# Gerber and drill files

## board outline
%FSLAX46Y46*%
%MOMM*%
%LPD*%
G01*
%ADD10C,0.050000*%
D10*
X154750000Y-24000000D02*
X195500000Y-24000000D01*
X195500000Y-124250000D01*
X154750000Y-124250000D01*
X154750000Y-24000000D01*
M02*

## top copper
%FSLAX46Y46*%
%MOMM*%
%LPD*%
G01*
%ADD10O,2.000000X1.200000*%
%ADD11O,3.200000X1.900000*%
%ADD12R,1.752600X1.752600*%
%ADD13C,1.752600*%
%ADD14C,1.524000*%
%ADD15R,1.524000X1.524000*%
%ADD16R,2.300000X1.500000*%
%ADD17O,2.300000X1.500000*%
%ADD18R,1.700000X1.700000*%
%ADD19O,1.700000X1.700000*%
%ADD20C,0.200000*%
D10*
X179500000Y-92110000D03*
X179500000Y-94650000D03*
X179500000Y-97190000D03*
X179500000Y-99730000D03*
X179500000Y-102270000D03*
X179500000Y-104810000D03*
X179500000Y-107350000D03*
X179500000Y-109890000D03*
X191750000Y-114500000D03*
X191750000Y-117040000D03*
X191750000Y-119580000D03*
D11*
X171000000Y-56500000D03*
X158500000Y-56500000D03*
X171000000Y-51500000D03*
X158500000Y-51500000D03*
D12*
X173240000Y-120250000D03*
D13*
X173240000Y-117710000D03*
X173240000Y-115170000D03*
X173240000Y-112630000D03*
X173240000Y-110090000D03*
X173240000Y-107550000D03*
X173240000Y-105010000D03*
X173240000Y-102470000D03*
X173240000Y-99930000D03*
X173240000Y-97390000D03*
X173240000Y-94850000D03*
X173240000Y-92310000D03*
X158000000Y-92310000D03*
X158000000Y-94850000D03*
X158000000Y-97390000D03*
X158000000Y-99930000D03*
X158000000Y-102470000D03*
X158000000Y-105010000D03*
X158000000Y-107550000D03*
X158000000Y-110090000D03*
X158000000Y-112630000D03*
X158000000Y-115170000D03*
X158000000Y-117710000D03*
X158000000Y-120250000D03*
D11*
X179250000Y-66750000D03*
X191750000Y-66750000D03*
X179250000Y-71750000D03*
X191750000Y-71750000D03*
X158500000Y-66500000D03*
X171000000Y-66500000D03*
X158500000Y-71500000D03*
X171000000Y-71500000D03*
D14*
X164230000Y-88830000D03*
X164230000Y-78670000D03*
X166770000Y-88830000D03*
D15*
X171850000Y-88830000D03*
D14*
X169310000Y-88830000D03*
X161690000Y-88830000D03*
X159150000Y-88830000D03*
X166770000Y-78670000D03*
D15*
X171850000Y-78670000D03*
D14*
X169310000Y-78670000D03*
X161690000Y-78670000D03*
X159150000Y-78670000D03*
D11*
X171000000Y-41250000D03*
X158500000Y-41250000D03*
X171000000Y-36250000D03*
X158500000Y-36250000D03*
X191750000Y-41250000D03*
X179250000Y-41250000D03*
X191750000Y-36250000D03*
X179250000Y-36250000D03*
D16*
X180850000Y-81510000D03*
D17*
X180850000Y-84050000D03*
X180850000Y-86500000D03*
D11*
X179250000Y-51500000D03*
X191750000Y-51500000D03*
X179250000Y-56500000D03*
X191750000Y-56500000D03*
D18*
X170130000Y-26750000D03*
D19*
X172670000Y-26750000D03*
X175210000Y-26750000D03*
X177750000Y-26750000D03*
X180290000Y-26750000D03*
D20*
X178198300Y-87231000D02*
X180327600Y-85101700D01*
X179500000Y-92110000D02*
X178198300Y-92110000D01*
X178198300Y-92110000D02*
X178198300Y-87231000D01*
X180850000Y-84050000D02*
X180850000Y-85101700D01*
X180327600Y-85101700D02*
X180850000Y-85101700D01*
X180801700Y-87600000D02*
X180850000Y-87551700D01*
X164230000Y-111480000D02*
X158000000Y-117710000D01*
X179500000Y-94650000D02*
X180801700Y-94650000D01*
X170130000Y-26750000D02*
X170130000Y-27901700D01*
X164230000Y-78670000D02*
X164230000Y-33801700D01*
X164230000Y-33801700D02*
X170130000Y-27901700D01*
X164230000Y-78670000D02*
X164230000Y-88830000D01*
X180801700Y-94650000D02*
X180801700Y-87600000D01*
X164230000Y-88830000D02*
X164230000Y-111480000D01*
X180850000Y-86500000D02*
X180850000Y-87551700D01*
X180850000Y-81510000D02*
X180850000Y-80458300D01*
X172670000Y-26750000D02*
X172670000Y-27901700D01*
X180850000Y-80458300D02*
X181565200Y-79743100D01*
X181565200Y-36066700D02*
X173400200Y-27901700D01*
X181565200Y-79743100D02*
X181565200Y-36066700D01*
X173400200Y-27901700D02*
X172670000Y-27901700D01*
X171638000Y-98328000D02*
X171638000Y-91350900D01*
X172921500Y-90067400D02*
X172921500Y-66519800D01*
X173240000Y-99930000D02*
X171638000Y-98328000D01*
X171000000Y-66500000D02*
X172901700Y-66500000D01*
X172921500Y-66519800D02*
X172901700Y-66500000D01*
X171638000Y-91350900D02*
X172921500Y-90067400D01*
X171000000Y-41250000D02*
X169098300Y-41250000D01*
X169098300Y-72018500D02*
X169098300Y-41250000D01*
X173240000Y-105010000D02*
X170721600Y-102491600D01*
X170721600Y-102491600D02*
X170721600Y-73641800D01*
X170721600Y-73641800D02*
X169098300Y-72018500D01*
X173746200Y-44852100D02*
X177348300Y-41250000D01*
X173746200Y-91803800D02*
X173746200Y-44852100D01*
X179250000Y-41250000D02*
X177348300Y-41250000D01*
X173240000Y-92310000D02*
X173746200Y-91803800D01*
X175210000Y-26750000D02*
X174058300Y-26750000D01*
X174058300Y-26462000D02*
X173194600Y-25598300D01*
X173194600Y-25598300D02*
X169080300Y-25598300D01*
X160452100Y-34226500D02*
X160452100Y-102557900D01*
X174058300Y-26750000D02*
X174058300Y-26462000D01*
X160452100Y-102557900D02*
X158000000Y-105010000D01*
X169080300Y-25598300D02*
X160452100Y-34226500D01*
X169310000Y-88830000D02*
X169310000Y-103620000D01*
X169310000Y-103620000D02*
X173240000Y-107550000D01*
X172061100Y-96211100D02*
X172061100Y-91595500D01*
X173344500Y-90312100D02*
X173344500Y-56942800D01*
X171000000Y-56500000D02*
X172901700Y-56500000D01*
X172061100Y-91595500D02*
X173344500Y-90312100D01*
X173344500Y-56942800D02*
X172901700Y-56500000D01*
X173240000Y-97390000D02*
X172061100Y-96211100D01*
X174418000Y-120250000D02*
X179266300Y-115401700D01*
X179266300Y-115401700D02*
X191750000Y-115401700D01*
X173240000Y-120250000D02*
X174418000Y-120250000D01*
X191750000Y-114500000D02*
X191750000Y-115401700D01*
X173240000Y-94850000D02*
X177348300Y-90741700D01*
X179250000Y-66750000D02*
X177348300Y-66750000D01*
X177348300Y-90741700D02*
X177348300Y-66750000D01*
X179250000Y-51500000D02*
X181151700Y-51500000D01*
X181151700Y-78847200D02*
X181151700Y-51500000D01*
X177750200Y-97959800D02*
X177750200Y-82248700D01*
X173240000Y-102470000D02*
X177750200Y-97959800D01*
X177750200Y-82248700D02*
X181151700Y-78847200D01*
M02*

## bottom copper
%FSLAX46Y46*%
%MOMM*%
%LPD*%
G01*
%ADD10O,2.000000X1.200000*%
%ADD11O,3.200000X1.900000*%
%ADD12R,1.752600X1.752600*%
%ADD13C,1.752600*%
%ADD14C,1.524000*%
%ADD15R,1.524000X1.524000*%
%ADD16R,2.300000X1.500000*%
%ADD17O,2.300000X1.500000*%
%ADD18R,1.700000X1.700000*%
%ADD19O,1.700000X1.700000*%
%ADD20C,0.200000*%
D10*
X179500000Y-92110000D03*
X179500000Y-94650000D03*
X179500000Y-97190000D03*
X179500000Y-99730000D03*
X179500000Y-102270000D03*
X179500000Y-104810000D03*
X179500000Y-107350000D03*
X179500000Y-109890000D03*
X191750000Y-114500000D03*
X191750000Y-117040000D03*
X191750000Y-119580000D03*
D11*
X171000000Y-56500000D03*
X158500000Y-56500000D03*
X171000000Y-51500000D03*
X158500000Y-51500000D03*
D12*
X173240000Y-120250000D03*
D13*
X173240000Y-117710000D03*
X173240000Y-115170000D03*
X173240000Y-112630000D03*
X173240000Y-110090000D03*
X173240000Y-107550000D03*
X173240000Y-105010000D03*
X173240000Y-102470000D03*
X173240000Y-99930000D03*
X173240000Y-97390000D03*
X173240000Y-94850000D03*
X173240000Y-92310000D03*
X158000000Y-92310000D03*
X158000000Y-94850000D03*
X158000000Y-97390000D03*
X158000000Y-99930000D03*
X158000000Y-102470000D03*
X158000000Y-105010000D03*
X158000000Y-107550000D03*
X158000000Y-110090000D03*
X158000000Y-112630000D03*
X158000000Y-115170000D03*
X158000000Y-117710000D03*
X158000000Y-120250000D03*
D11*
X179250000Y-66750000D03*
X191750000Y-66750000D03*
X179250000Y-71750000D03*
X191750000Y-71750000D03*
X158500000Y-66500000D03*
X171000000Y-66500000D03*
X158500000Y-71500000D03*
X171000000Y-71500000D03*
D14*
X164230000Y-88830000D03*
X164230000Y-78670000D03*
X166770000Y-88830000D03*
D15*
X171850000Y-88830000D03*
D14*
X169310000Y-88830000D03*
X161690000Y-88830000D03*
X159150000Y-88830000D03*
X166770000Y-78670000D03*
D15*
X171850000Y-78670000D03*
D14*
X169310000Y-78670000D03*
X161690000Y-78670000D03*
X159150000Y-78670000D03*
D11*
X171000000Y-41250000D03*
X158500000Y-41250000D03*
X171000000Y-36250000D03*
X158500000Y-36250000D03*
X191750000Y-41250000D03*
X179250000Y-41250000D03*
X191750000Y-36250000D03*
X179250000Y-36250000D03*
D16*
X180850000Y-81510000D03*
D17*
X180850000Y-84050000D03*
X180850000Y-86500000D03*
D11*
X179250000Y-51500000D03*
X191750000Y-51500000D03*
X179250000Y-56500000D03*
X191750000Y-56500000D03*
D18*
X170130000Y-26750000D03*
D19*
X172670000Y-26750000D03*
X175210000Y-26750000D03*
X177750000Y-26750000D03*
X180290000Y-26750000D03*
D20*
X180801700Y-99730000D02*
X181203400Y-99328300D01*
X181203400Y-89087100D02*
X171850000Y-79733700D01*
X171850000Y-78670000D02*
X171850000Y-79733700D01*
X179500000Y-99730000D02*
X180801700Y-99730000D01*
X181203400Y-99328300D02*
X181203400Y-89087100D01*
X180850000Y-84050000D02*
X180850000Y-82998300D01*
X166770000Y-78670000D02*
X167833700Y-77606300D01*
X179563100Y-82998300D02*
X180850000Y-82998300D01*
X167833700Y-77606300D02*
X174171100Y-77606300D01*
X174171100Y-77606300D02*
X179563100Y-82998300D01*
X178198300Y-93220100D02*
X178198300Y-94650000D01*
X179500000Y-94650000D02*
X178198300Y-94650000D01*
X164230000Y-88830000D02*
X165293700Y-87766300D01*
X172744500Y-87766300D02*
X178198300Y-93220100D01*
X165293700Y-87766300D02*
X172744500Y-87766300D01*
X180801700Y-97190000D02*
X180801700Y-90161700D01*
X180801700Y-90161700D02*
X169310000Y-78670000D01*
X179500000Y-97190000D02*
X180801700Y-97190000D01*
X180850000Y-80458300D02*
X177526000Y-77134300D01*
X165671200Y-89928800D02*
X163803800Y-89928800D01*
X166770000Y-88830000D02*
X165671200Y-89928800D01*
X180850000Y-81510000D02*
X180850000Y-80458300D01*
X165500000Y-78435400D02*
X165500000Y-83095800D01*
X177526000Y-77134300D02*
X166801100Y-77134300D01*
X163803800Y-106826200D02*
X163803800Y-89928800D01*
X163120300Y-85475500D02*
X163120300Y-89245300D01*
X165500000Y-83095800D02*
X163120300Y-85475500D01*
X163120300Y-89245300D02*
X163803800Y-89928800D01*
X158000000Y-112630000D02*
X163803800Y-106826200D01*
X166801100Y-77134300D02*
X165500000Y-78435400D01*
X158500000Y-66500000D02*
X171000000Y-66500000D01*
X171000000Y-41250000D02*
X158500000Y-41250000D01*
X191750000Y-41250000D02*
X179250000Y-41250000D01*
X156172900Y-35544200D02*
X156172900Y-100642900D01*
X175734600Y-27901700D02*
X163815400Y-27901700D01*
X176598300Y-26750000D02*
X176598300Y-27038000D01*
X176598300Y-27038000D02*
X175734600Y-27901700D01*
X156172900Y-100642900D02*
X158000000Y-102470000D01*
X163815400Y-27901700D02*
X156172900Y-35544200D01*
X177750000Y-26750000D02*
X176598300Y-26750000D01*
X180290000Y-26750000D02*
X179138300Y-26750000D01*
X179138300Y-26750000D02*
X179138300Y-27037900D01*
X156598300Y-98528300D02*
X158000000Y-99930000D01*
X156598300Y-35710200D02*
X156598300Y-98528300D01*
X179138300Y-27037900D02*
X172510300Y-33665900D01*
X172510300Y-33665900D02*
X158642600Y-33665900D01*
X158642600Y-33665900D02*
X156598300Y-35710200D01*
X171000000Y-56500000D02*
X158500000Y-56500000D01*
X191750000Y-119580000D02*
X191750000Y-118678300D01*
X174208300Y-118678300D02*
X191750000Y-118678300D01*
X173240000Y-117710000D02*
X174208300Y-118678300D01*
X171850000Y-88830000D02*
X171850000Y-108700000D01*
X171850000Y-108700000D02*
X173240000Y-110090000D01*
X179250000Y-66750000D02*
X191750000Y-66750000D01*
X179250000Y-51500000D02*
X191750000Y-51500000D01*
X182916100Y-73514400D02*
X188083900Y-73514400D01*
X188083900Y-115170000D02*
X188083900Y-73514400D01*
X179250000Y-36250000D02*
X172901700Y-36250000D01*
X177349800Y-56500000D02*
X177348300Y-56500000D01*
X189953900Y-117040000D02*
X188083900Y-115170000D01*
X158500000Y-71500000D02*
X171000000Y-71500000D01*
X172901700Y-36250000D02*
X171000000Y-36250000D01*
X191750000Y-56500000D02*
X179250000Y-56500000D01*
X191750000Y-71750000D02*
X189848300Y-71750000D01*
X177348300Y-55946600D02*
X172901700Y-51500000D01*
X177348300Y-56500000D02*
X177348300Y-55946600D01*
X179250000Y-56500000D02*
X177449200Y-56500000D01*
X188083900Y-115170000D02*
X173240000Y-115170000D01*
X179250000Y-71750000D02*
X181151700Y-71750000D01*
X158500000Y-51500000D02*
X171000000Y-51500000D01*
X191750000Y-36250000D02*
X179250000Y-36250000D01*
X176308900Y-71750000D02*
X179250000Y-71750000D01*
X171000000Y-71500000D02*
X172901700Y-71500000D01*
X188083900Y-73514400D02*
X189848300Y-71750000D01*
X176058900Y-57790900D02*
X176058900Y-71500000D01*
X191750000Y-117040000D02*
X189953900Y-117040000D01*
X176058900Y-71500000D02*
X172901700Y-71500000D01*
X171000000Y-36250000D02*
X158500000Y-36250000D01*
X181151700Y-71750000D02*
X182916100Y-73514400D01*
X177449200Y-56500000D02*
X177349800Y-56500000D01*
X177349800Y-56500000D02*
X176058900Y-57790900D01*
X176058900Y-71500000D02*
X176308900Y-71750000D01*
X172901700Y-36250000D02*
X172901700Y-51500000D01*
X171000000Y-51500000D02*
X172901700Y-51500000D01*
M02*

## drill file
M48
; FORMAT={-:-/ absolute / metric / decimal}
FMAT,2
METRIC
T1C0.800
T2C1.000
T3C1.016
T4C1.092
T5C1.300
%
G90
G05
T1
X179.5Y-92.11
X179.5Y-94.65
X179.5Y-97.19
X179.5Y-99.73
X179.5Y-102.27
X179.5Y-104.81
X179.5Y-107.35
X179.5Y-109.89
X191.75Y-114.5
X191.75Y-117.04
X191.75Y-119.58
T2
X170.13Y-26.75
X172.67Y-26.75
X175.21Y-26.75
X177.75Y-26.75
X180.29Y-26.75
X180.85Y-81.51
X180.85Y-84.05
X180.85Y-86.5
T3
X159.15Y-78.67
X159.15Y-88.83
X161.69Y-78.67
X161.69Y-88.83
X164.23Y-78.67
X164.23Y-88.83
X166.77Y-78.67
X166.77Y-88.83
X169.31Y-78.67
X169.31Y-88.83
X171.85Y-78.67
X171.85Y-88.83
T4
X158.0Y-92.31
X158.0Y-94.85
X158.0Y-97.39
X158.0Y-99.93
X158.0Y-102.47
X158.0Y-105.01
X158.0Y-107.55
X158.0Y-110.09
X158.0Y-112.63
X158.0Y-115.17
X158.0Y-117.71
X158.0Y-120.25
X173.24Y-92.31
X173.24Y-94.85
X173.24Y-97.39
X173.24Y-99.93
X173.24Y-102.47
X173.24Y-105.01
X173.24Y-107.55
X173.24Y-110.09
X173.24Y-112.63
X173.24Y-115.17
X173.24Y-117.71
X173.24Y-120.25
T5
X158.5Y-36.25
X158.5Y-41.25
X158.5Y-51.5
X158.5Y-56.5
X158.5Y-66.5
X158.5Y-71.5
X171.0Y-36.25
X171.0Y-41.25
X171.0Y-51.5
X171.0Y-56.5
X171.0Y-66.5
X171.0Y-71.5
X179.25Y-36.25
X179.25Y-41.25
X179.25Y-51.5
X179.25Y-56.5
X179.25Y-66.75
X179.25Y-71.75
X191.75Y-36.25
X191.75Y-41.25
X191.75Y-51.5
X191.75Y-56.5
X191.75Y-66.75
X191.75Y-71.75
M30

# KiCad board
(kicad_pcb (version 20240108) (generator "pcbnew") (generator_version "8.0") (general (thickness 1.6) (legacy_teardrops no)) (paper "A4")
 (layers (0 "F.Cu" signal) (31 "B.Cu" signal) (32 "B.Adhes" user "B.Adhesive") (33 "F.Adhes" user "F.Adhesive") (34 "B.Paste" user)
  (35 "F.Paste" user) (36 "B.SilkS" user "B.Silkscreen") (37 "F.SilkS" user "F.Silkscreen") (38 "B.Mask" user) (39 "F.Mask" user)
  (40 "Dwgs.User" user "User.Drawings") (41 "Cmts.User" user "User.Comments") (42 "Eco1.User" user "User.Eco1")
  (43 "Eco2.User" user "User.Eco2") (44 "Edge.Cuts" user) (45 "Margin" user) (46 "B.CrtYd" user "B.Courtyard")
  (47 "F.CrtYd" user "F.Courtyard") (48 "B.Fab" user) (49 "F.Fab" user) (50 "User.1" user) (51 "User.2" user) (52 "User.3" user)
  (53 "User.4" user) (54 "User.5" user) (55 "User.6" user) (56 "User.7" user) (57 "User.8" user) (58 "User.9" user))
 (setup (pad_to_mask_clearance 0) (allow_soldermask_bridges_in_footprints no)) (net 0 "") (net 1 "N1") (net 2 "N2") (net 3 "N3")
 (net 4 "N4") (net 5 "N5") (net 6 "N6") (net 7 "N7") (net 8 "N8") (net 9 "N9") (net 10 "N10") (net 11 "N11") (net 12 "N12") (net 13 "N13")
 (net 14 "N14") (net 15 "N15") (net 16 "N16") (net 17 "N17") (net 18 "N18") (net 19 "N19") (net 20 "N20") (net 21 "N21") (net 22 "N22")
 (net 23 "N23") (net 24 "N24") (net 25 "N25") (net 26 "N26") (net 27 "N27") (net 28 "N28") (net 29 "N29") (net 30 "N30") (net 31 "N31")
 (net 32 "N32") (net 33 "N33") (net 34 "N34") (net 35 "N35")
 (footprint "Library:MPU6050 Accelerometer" (layer "F.Cu") (at 186 103.25)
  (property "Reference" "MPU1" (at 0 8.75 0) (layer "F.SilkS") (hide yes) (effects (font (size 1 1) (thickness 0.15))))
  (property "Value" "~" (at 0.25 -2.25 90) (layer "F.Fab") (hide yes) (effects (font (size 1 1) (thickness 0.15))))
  (pad "1" thru_hole oval (at -6.5 -11.14 270) (size 1.2 2) (drill 0.8) (layers "*.Cu" "*.Mask") (remove_unused_layers no) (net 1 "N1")
   (thermal_bridge_angle 45))
  (pad "2" thru_hole oval (at -6.5 -8.6 270) (size 1.2 2) (drill 0.8) (layers "*.Cu" "*.Mask") (remove_unused_layers no) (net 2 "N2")
   (thermal_bridge_angle 45))
  (pad "3" thru_hole oval (at -6.5 -6.06 270) (size 1.2 2) (drill 0.8) (layers "*.Cu" "*.Mask") (remove_unused_layers no) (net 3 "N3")
   (thermal_bridge_angle 45))
  (pad "4" thru_hole oval (at -6.5 -3.52 270) (size 1.2 2) (drill 0.8) (layers "*.Cu" "*.Mask") (remove_unused_layers no) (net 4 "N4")
   (thermal_bridge_angle 45))
  (pad "5" thru_hole oval (at -6.5 -0.98 270) (size 1.2 2) (drill 0.8) (layers "*.Cu" "*.Mask") (remove_unused_layers no) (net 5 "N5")
   (thermal_bridge_angle 45))
  (pad "6" thru_hole oval (at -6.5 1.56 270) (size 1.2 2) (drill 0.8) (layers "*.Cu" "*.Mask") (remove_unused_layers no) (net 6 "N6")
   (thermal_bridge_angle 45))
  (pad "7" thru_hole oval (at -6.5 4.1 270) (size 1.2 2) (drill 0.8) (layers "*.Cu" "*.Mask") (remove_unused_layers no) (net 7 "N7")
   (thermal_bridge_angle 45))
  (pad "8" thru_hole oval (at -6.5 6.64 270) (size 1.2 2) (drill 0.8) (layers "*.Cu" "*.Mask") (remove_unused_layers no) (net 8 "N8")
   (thermal_bridge_angle 45)))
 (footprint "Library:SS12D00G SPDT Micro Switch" (layer "F.Cu") (at 191.75 117.04 -90)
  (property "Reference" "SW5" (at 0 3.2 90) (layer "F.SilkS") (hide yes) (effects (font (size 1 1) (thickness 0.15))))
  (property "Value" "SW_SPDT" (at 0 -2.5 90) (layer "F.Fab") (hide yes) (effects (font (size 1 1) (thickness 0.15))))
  (pad "1" thru_hole oval (at -2.54 0 270) (size 1.2 2) (drill 0.8) (layers "*.Cu" "*.Mask") (remove_unused_layers no) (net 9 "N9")
   (thermal_bridge_angle 45))
  (pad "2" thru_hole oval (at 0 0 270) (size 1.2 2) (drill 0.8) (layers "*.Cu" "*.Mask") (remove_unused_layers no) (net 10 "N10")
   (thermal_bridge_angle 45))
  (pad "3" thru_hole oval (at 2.54 0 270) (size 1.2 2) (drill 0.8) (layers "*.Cu" "*.Mask") (remove_unused_layers no) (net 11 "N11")
   (thermal_bridge_angle 45)))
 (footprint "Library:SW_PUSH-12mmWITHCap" (layer "F.Cu") (at 171 56.5 180)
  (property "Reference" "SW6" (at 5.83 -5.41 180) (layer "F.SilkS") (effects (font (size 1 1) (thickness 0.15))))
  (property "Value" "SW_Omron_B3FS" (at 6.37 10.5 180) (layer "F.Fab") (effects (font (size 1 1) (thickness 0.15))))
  (pad "1" thru_hole oval (at 0 0 180) (size 3.2 1.9) (drill 1.3) (layers "*.Cu" "*.Mask") (remove_unused_layers no) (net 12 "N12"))
  (pad "1" thru_hole oval (at 12.5 0 180) (size 3.2 1.9) (drill 1.3) (layers "*.Cu" "*.Mask") (remove_unused_layers no) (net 12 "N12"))
  (pad "2" thru_hole oval (at 0 5 180) (size 3.2 1.9) (drill 1.3) (layers "*.Cu" "*.Mask") (remove_unused_layers no) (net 10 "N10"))
  (pad "2" thru_hole oval (at 12.5 5 180) (size 3.2 1.9) (drill 1.3) (layers "*.Cu" "*.Mask") (remove_unused_layers no) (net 10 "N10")))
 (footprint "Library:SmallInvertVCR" (layer "F.Cu") (at 182.25 117.5)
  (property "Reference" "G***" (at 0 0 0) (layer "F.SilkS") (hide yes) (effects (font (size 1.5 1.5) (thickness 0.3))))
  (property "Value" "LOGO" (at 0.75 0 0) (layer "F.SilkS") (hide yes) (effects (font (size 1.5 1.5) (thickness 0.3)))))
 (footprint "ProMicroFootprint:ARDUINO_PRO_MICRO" (layer "F.Cu") (at 165.62 106.28 90)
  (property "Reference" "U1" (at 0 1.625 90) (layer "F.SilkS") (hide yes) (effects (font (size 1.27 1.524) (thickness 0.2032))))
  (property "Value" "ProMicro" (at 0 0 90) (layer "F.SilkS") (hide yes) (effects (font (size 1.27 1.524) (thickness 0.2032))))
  (pad "1" thru_hole rect (at -13.97 7.62 90) (size 1.7526 1.7526) (drill 1.0922) (layers "*.Cu" "*.SilkS" "*.Mask")
   (remove_unused_layers no) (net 9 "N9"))
  (pad "2" thru_hole circle (at -11.43 7.62 90) (size 1.7526 1.7526) (drill 1.0922) (layers "*.Cu" "*.SilkS" "*.Mask")
   (remove_unused_layers no) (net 11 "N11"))
  (pad "3" thru_hole circle (at -8.89 7.62 90) (size 1.7526 1.7526) (drill 1.0922) (layers "*.Cu" "*.SilkS" "*.Mask")
   (remove_unused_layers no) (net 10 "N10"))
  (pad "4" thru_hole circle (at -6.35 7.62 90) (size 1.7526 1.7526) (drill 1.0922) (layers "*.Cu" "*.SilkS" "*.Mask")
   (remove_unused_layers no) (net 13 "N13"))
  (pad "5" thru_hole circle (at -3.81 7.62 90) (size 1.7526 1.7526) (drill 1.0922) (layers "*.Cu" "*.SilkS" "*.Mask")
   (remove_unused_layers no) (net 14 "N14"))
  (pad "6" thru_hole circle (at -1.27 7.62 90) (size 1.7526 1.7526) (drill 1.0922) (layers "*.Cu" "*.SilkS" "*.Mask")
   (remove_unused_layers no) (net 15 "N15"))
  (pad "7" thru_hole circle (at 1.27 7.62 90) (size 1.7526 1.7526) (drill 1.0922) (layers "*.Cu" "*.SilkS" "*.Mask")
   (remove_unused_layers no) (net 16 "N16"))
  (pad "8" thru_hole circle (at 3.81 7.62 90) (size 1.7526 1.7526) (drill 1.0922) (layers "*.Cu" "*.SilkS" "*.Mask")
   (remove_unused_layers no) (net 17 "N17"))
  (pad "9" thru_hole circle (at 6.35 7.62 90) (size 1.7526 1.7526) (drill 1.0922) (layers "*.Cu" "*.SilkS" "*.Mask")
   (remove_unused_layers no) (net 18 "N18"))
  (pad "10" thru_hole circle (at 8.89 7.62 90) (size 1.7526 1.7526) (drill 1.0922) (layers "*.Cu" "*.SilkS" "*.Mask")
   (remove_unused_layers no) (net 12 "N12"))
  (pad "11" thru_hole circle (at 11.43 7.62 90) (size 1.7526 1.7526) (drill 1.0922) (layers "*.Cu" "*.SilkS" "*.Mask")
   (remove_unused_layers no) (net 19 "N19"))
  (pad "12" thru_hole circle (at 13.97 7.62 90) (size 1.7526 1.7526) (drill 1.0922) (layers "*.Cu" "*.SilkS" "*.Mask")
   (remove_unused_layers no) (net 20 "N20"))
  (pad "13" thru_hole circle (at 13.97 -7.62 90) (size 1.7526 1.7526) (drill 1.0922) (layers "*.Cu" "*.SilkS" "*.Mask")
   (remove_unused_layers no) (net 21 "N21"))
  (pad "14" thru_hole circle (at 11.43 -7.62 90) (size 1.7526 1.7526) (drill 1.0922) (layers "*.Cu" "*.SilkS" "*.Mask")
   (remove_unused_layers no) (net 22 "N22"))
  (pad "15" thru_hole circle (at 8.89 -7.62 90) (size 1.7526 1.7526) (drill 1.0922) (layers "*.Cu" "*.SilkS" "*.Mask")
   (remove_unused_layers no) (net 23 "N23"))
  (pad "16" thru_hole circle (at 6.35 -7.62 90) (size 1.7526 1.7526) (drill 1.0922) (layers "*.Cu" "*.SilkS" "*.Mask")
   (remove_unused_layers no) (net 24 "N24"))
  (pad "17" thru_hole circle (at 3.81 -7.62 90) (size 1.7526 1.7526) (drill 1.0922) (layers "*.Cu" "*.SilkS" "*.Mask")
   (remove_unused_layers no) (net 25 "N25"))
  (pad "18" thru_hole circle (at 1.27 -7.62 90) (size 1.7526 1.7526) (drill 1.0922) (layers "*.Cu" "*.SilkS" "*.Mask")
   (remove_unused_layers no) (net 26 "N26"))
  (pad "19" thru_hole circle (at -1.27 -7.62 90) (size 1.7526 1.7526) (drill 1.0922) (layers "*.Cu" "*.SilkS" "*.Mask")
   (remove_unused_layers no) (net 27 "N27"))
  (pad "20" thru_hole circle (at -3.81 -7.62 90) (size 1.7526 1.7526) (drill 1.0922) (layers "*.Cu" "*.SilkS" "*.Mask")
   (remove_unused_layers no) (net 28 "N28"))
  (pad "21" thru_hole circle (at -6.35 -7.62 90) (size 1.7526 1.7526) (drill 1.0922) (layers "*.Cu" "*.SilkS" "*.Mask")
   (remove_unused_layers no) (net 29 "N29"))
  (pad "22" thru_hole circle (at -8.89 -7.62 90) (size 1.7526 1.7526) (drill 1.0922) (layers "*.Cu" "*.SilkS" "*.Mask")
   (remove_unused_layers no) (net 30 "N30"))
  (pad "23" thru_hole circle (at -11.43 -7.62 90) (size 1.7526 1.7526) (drill 1.0922) (layers "*.Cu" "*.SilkS" "*.Mask")
   (remove_unused_layers no) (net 2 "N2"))
  (pad "24" thru_hole circle (at -13.97 -7.62 90) (size 1.7526 1.7526) (drill 1.0922) (layers "*.Cu" "*.SilkS" "*.Mask")
   (remove_unused_layers no) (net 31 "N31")))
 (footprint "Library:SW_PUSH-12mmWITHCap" (layer "F.Cu") (at 179.25 66.75)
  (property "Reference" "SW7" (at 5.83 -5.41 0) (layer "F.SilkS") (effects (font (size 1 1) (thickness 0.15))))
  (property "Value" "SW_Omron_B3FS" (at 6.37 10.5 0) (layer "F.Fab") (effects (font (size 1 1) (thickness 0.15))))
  (pad "1" thru_hole oval (at 0 0) (size 3.2 1.9) (drill 1.3) (layers "*.Cu" "*.Mask") (remove_unused_layers no) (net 19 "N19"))
  (pad "1" thru_hole oval (at 12.5 0) (size 3.2 1.9) (drill 1.3) (layers "*.Cu" "*.Mask") (remove_unused_layers no) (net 19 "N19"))
  (pad "2" thru_hole oval (at 0 5) (size 3.2 1.9) (drill 1.3) (layers "*.Cu" "*.Mask") (remove_unused_layers no) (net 10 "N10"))
  (pad "2" thru_hole oval (at 12.5 5) (size 3.2 1.9) (drill 1.3) (layers "*.Cu" "*.Mask") (remove_unused_layers no) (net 10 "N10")))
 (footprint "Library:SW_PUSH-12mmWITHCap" (layer "F.Cu") (at 158.5 66.5)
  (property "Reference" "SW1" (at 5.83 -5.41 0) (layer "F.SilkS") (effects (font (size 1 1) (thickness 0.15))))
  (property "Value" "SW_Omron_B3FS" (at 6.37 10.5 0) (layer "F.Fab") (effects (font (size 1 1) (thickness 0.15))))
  (pad "1" thru_hole oval (at 0 0) (size 3.2 1.9) (drill 1.3) (layers "*.Cu" "*.Mask") (remove_unused_layers no) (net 18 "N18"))
  (pad "1" thru_hole oval (at 12.5 0) (size 3.2 1.9) (drill 1.3) (layers "*.Cu" "*.Mask") (remove_unused_layers no) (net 18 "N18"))
  (pad "2" thru_hole oval (at 0 5) (size 3.2 1.9) (drill 1.3) (layers "*.Cu" "*.Mask") (remove_unused_layers no) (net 10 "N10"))
  (pad "2" thru_hole oval (at 12.5 5) (size 3.2 1.9) (drill 1.3) (layers "*.Cu" "*.Mask") (remove_unused_layers no) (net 10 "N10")))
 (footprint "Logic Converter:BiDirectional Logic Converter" (layer "F.Cu") (at 165.5 83.75 -90)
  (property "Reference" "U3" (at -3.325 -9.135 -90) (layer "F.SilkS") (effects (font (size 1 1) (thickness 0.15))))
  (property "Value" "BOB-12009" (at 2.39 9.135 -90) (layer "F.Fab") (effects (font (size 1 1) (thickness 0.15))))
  (pad "GND_1" thru_hole circle (at 5.08 1.27 270) (size 1.524 1.524) (drill 1.016) (layers "*.Cu" "*.Mask") (remove_unused_layers no)
   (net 2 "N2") (solder_mask_margin 0.102))
  (pad "GND_2" thru_hole circle (at -5.08 1.27 270) (size 1.524 1.524) (drill 1.016) (layers "*.Cu" "*.Mask") (remove_unused_layers no)
   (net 2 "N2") (solder_mask_margin 0.102))
  (pad "HV" thru_hole circle (at 5.08 -1.27 270) (size 1.524 1.524) (drill 1.016) (layers "*.Cu" "*.Mask") (remove_unused_layers no)
   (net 29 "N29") (solder_mask_margin 0.102))
  (pad "HV1" thru_hole rect (at 5.08 -6.35 270) (size 1.524 1.524) (drill 1.016) (layers "*.Cu" "*.Mask") (remove_unused_layers no)
   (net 14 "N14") (solder_mask_margin 0.102))
  (pad "HV2" thru_hole circle (at 5.08 -3.81 270) (size 1.524 1.524) (drill 1.016) (layers "*.Cu" "*.Mask") (remove_unused_layers no)
   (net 15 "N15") (solder_mask_margin 0.102))
  (pad "HV3" thru_hole circle (at 5.08 3.81 270) (size 1.524 1.524) (drill 1.016) (layers "*.Cu" "*.Mask") (remove_unused_layers no)
   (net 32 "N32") (solder_mask_margin 0.102))
  (pad "HV4" thru_hole circle (at 5.08 6.35 270) (size 1.524 1.524) (drill 1.016) (layers "*.Cu" "*.Mask") (remove_unused_layers no)
   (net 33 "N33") (solder_mask_margin 0.102))
  (pad "LV" thru_hole circle (at -5.08 -1.27 270) (size 1.524 1.524) (drill 1.016) (layers "*.Cu" "*.Mask") (remove_unused_layers no)
   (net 1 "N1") (solder_mask_margin 0.102))
  (pad "LV1" thru_hole rect (at -5.08 -6.35 270) (size 1.524 1.524) (drill 1.016) (layers "*.Cu" "*.Mask") (remove_unused_layers no)
   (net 4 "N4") (solder_mask_margin 0.102))
  (pad "LV2" thru_hole circle (at -5.08 -3.81 270) (size 1.524 1.524) (drill 1.016) (layers "*.Cu" "*.Mask") (remove_unused_layers no)
   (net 3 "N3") (solder_mask_margin 0.102))
  (pad "LV3" thru_hole circle (at -5.08 3.81 270) (size 1.524 1.524) (drill 1.016) (layers "*.Cu" "*.Mask") (remove_unused_layers no)
   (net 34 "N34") (solder_mask_margin 0.102))
  (pad "LV4" thru_hole circle (at -5.08 6.35 270) (size 1.524 1.524) (drill 1.016) (layers "*.Cu" "*.Mask") (remove_unused_layers no)
   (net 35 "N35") (solder_mask_margin 0.102)))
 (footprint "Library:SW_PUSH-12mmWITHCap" (layer "F.Cu") (at 171 41.25 180)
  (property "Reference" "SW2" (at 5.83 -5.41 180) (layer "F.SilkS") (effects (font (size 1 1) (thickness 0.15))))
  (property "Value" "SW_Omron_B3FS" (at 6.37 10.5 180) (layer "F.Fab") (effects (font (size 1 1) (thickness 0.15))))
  (pad "1" thru_hole oval (at 0 0 180) (size 3.2 1.9) (drill 1.3) (layers "*.Cu" "*.Mask") (remove_unused_layers no) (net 16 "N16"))
  (pad "1" thru_hole oval (at 12.5 0 180) (size 3.2 1.9) (drill 1.3) (layers "*.Cu" "*.Mask") (remove_unused_layers no) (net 16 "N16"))
  (pad "2" thru_hole oval (at 0 5 180) (size 3.2 1.9) (drill 1.3) (layers "*.Cu" "*.Mask") (remove_unused_layers no) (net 10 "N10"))
  (pad "2" thru_hole oval (at 12.5 5 180) (size 3.2 1.9) (drill 1.3) (layers "*.Cu" "*.Mask") (remove_unused_layers no) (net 10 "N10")))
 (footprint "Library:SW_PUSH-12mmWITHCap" (layer "F.Cu") (at 191.75 41.25 180)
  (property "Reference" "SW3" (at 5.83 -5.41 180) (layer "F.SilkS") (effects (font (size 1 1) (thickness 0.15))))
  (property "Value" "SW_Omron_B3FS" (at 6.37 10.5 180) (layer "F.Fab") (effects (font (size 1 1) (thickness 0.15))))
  (pad "1" thru_hole oval (at 0 0 180) (size 3.2 1.9) (drill 1.3) (layers "*.Cu" "*.Mask") (remove_unused_layers no) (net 20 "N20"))
  (pad "1" thru_hole oval (at 12.5 0 180) (size 3.2 1.9) (drill 1.3) (layers "*.Cu" "*.Mask") (remove_unused_layers no) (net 20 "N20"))
  (pad "2" thru_hole oval (at 0 5 180) (size 3.2 1.9) (drill 1.3) (layers "*.Cu" "*.Mask") (remove_unused_layers no) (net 10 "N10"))
  (pad "2" thru_hole oval (at 12.5 5 180) (size 3.2 1.9) (drill 1.3) (layers "*.Cu" "*.Mask") (remove_unused_layers no) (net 10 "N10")))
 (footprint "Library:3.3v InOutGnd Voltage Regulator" (layer "F.Cu") (at 179.35 84 -90)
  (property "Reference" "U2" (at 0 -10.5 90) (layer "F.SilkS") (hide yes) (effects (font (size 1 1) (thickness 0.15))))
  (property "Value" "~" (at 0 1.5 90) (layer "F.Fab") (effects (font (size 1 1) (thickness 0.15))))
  (pad "1" thru_hole rect (at -2.49 -1.5 270) (size 1.5 2.3) (drill 1) (layers "*.Cu" "*.Mask") (remove_unused_layers no) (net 29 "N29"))
  (pad "2" thru_hole oval (at 0.05 -1.5 270) (size 1.5 2.3) (drill 1) (layers "*.Cu" "*.Mask") (remove_unused_layers no) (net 1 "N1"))
  (pad "3" thru_hole oval (at 2.5 -1.5 270) (size 1.5 2.3) (drill 1) (layers "*.Cu" "*.Mask") (remove_unused_layers no) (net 2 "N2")))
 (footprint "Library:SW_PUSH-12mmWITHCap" (layer "F.Cu") (at 179.25 51.5)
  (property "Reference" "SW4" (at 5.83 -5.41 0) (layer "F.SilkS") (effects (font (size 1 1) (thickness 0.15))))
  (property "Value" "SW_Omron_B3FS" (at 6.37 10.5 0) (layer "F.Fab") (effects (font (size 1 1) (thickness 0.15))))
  (pad "1" thru_hole oval (at 0 0) (size 3.2 1.9) (drill 1.3) (layers "*.Cu" "*.Mask") (remove_unused_layers no) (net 17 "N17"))
  (pad "1" thru_hole oval (at 12.5 0) (size 3.2 1.9) (drill 1.3) (layers "*.Cu" "*.Mask") (remove_unused_layers no) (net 17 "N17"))
  (pad "2" thru_hole oval (at 0 5) (size 3.2 1.9) (drill 1.3) (layers "*.Cu" "*.Mask") (remove_unused_layers no) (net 10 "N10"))
  (pad "2" thru_hole oval (at 12.5 5) (size 3.2 1.9) (drill 1.3) (layers "*.Cu" "*.Mask") (remove_unused_layers no) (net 10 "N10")))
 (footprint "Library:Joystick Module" (layer "B.Cu") (at 170.13 26.75 -90)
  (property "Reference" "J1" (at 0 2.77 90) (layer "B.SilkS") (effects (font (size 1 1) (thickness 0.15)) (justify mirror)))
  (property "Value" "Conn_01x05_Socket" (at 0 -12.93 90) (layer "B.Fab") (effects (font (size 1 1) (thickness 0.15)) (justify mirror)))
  (pad "1" thru_hole rect (at 0 0 270) (size 1.7 1.7) (drill 1) (layers "*.Cu" "*.Mask") (remove_unused_layers no) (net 2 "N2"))
  (pad "2" thru_hole oval (at 0 -2.54 270) (size 1.7 1.7) (drill 1) (layers "*.Cu" "*.Mask") (remove_unused_layers no) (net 29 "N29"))
  (pad "3" thru_hole oval (at 0 -5.08 270) (size 1.7 1.7) (drill 1) (layers "*.Cu" "*.Mask") (remove_unused_layers no) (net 26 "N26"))
  (pad "4" thru_hole oval (at 0 -7.62 270) (size 1.7 1.7) (drill 1) (layers "*.Cu" "*.Mask") (remove_unused_layers no) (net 25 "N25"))
  (pad "5" thru_hole oval (at 0 -10.16 270) (size 1.7 1.7) (drill 1) (layers "*.Cu" "*.Mask") (remove_unused_layers no) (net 24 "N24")))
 (gr_rect (start 154.75 24) (end 195.5 124.25) (stroke (width 0.05) (type default)) (fill none) (layer "Edge.Cuts"))
 (segment (start 180.8017 99.73) (end 181.2034 99.3283) (width 0.2) (layer "B.Cu") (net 4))
 (segment (start 181.2034 89.0871) (end 171.85 79.7337) (width 0.2) (layer "B.Cu") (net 4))
 (segment (start 171.85 78.67) (end 171.85 79.7337) (width 0.2) (layer "B.Cu") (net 4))
 (segment (start 179.5 99.73) (end 180.8017 99.73) (width 0.2) (layer "B.Cu") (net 4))
 (segment (start 181.2034 99.3283) (end 181.2034 89.0871) (width 0.2) (layer "B.Cu") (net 4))
 (segment (start 178.1983 87.231) (end 180.3276 85.1017) (width 0.2) (layer "F.Cu") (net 1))
 (segment (start 179.5 92.11) (end 178.1983 92.11) (width 0.2) (layer "F.Cu") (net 1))
 (segment (start 178.1983 92.11) (end 178.1983 87.231) (width 0.2) (layer "F.Cu") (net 1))
 (segment (start 180.85 84.05) (end 180.85 85.1017) (width 0.2) (layer "F.Cu") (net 1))
 (segment (start 180.3276 85.1017) (end 180.85 85.1017) (width 0.2) (layer "F.Cu") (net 1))
 (segment (start 180.85 84.05) (end 180.85 82.9983) (width 0.2) (layer "B.Cu") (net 1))
 (segment (start 166.77 78.67) (end 167.8337 77.6063) (width 0.2) (layer "B.Cu") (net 1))
 (segment (start 179.5631 82.9983) (end 180.85 82.9983) (width 0.2) (layer "B.Cu") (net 1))
 (segment (start 167.8337 77.6063) (end 174.1711 77.6063) (width 0.2) (layer "B.Cu") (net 1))
 (segment (start 174.1711 77.6063) (end 179.5631 82.9983) (width 0.2) (layer "B.Cu") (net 1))
 (segment (start 180.8017 87.6) (end 180.85 87.5517) (width 0.2) (layer "F.Cu") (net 2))
 (segment (start 164.23 111.48) (end 158 117.71) (width 0.2) (layer "F.Cu") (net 2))
 (segment (start 179.5 94.65) (end 180.8017 94.65) (width 0.2) (layer "F.Cu") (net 2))
 (segment (start 170.13 26.75) (end 170.13 27.9017) (width 0.2) (layer "F.Cu") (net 2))
 (segment (start 164.23 78.67) (end 164.23 33.8017) (width 0.2) (layer "F.Cu") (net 2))
 (segment (start 164.23 33.8017) (end 170.13 27.9017) (width 0.2) (layer "F.Cu") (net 2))
 (segment (start 164.23 78.67) (end 164.23 88.83) (width 0.2) (layer "F.Cu") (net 2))
 (segment (start 180.8017 94.65) (end 180.8017 87.6) (width 0.2) (layer "F.Cu") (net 2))
 (segment (start 164.23 88.83) (end 164.23 111.48) (width 0.2) (layer "F.Cu") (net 2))
 (segment (start 180.85 86.5) (end 180.85 87.5517) (width 0.2) (layer "F.Cu") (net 2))
 (segment (start 178.1983 93.2201) (end 178.1983 94.65) (width 0.2) (layer "B.Cu") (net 2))
 (segment (start 179.5 94.65) (end 178.1983 94.65) (width 0.2) (layer "B.Cu") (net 2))
 (segment (start 164.23 88.83) (end 165.2937 87.7663) (width 0.2) (layer "B.Cu") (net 2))
 (segment (start 172.7445 87.7663) (end 178.1983 93.2201) (width 0.2) (layer "B.Cu") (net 2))
 (segment (start 165.2937 87.7663) (end 172.7445 87.7663) (width 0.2) (layer "B.Cu") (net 2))
 (segment (start 180.8017 97.19) (end 180.8017 90.1617) (width 0.2) (layer "B.Cu") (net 3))
 (segment (start 180.8017 90.1617) (end 169.31 78.67) (width 0.2) (layer "B.Cu") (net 3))
 (segment (start 179.5 97.19) (end 180.8017 97.19) (width 0.2) (layer "B.Cu") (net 3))
 (segment (start 180.85 81.51) (end 180.85 80.4583) (width 0.2) (layer "F.Cu") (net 29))
 (segment (start 172.67 26.75) (end 172.67 27.9017) (width 0.2) (layer "F.Cu") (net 29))
 (segment (start 180.85 80.4583) (end 181.5652 79.7431) (width 0.2) (layer "F.Cu") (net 29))
 (segment (start 181.5652 36.0667) (end 173.4002 27.9017) (width 0.2) (layer "F.Cu") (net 29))
 (segment (start 181.5652 79.7431) (end 181.5652 36.0667) (width 0.2) (layer "F.Cu") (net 29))
 (segment (start 173.4002 27.9017) (end 172.67 27.9017) (width 0.2) (layer "F.Cu") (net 29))
 (segment (start 180.85 80.4583) (end 177.526 77.1343) (width 0.2) (layer "B.Cu") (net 29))
 (segment (start 165.6712 89.9288) (end 163.8038 89.9288) (width 0.2) (layer "B.Cu") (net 29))
 (segment (start 166.77 88.83) (end 165.6712 89.9288) (width 0.2) (layer "B.Cu") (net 29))
 (segment (start 180.85 81.51) (end 180.85 80.4583) (width 0.2) (layer "B.Cu") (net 29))
 (segment (start 165.5 78.4354) (end 165.5 83.0958) (width 0.2) (layer "B.Cu") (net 29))
 (segment (start 177.526 77.1343) (end 166.8011 77.1343) (width 0.2) (layer "B.Cu") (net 29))
 (segment (start 163.8038 106.8262) (end 163.8038 89.9288) (width 0.2) (layer "B.Cu") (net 29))
 (segment (start 163.1203 85.4755) (end 163.1203 89.2453) (width 0.2) (layer "B.Cu") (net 29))
 (segment (start 165.5 83.0958) (end 163.1203 85.4755) (width 0.2) (layer "B.Cu") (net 29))
 (segment (start 163.1203 89.2453) (end 163.8038 89.9288) (width 0.2) (layer "B.Cu") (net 29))
 (segment (start 158 112.63) (end 163.8038 106.8262) (width 0.2) (layer "B.Cu") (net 29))
 (segment (start 166.8011 77.1343) (end 165.5 78.4354) (width 0.2) (layer "B.Cu") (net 29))
 (segment (start 171.638 98.328) (end 171.638 91.3509) (width 0.2) (layer "F.Cu") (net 18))
 (segment (start 172.9215 90.0674) (end 172.9215 66.5198) (width 0.2) (layer "F.Cu") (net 18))
 (segment (start 173.24 99.93) (end 171.638 98.328) (width 0.2) (layer "F.Cu") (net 18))
 (segment (start 171 66.5) (end 172.9017 66.5) (width 0.2) (layer "F.Cu") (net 18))
 (segment (start 172.9215 66.5198) (end 172.9017 66.5) (width 0.2) (layer "F.Cu") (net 18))
 (segment (start 171.638 91.3509) (end 172.9215 90.0674) (width 0.2) (layer "F.Cu") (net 18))
 (segment (start 158.5 66.5) (end 171 66.5) (width 0.2) (layer "B.Cu") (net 18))
 (segment (start 171 41.25) (end 169.0983 41.25) (width 0.2) (layer "F.Cu") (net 16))
 (segment (start 169.0983 72.0185) (end 169.0983 41.25) (width 0.2) (layer "F.Cu") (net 16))
 (segment (start 173.24 105.01) (end 170.7216 102.4916) (width 0.2) (layer "F.Cu") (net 16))
 (segment (start 170.7216 102.4916) (end 170.7216 73.6418) (width 0.2) (layer "F.Cu") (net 16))
 (segment (start 170.7216 73.6418) (end 169.0983 72.0185) (width 0.2) (layer "F.Cu") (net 16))
 (segment (start 171 41.25) (end 158.5 41.25) (width 0.2) (layer "B.Cu") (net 16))
 (segment (start 173.7462 44.8521) (end 177.3483 41.25) (width 0.2) (layer "F.Cu") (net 20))
 (segment (start 173.7462 91.8038) (end 173.7462 44.8521) (width 0.2) (layer "F.Cu") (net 20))
 (segment (start 179.25 41.25) (end 177.3483 41.25) (width 0.2) (layer "F.Cu") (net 20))
 (segment (start 173.24 92.31) (end 173.7462 91.8038) (width 0.2) (layer "F.Cu") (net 20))
 (segment (start 191.75 41.25) (end 179.25 41.25) (width 0.2) (layer "B.Cu") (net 20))
 (segment (start 156.1729 35.5442) (end 156.1729 100.6429) (width 0.2) (layer "B.Cu") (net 25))
 (segment (start 175.7346 27.9017) (end 163.8154 27.9017) (width 0.2) (layer "B.Cu") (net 25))
 (segment (start 176.5983 26.75) (end 176.5983 27.038) (width 0.2) (layer "B.Cu") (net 25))
 (segment (start 176.5983 27.038) (end 175.7346 27.9017) (width 0.2) (layer "B.Cu") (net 25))
 (segment (start 156.1729 100.6429) (end 158 102.47) (width 0.2) (layer "B.Cu") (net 25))
 (segment (start 163.8154 27.9017) (end 156.1729 35.5442) (width 0.2) (layer "B.Cu") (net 25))
 (segment (start 177.75 26.75) (end 176.5983 26.75) (width 0.2) (layer "B.Cu") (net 25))
 (segment (start 180.29 26.75) (end 179.1383 26.75) (width 0.2) (layer "B.Cu") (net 24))
 (segment (start 179.1383 26.75) (end 179.1383 27.0379) (width 0.2) (layer "B.Cu") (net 24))
 (segment (start 156.5983 98.5283) (end 158 99.93) (width 0.2) (layer "B.Cu") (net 24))
 (segment (start 156.5983 35.7102) (end 156.5983 98.5283) (width 0.2) (layer "B.Cu") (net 24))
 (segment (start 179.1383 27.0379) (end 172.5103 33.6659) (width 0.2) (layer "B.Cu") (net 24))
 (segment (start 172.5103 33.6659) (end 158.6426 33.6659) (width 0.2) (layer "B.Cu") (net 24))
 (segment (start 158.6426 33.6659) (end 156.5983 35.7102) (width 0.2) (layer "B.Cu") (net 24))
 (segment (start 175.21 26.75) (end 174.0583 26.75) (width 0.2) (layer "F.Cu") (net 26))
 (segment (start 174.0583 26.462) (end 173.1946 25.5983) (width 0.2) (layer "F.Cu") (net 26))
 (segment (start 173.1946 25.5983) (end 169.0803 25.5983) (width 0.2) (layer "F.Cu") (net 26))
 (segment (start 160.4521 34.2265) (end 160.4521 102.5579) (width 0.2) (layer "F.Cu") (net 26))
 (segment (start 174.0583 26.75) (end 174.0583 26.462) (width 0.2) (layer "F.Cu") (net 26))
 (segment (start 160.4521 102.5579) (end 158 105.01) (width 0.2) (layer "F.Cu") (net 26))
 (segment (start 169.0803 25.5983) (end 160.4521 34.2265) (width 0.2) (layer "F.Cu") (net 26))
 (segment (start 169.31 88.83) (end 169.31 103.62) (width 0.2) (layer "F.Cu") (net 15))
 (segment (start 169.31 103.62) (end 173.24 107.55) (width 0.2) (layer "F.Cu") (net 15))
 (segment (start 172.0611 96.2111) (end 172.0611 91.5955) (width 0.2) (layer "F.Cu") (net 12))
 (segment (start 173.3445 90.3121) (end 173.3445 56.9428) (width 0.2) (layer "F.Cu") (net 12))
 (segment (start 171 56.5) (end 172.9017 56.5) (width 0.2) (layer "F.Cu") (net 12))
 (segment (start 172.0611 91.5955) (end 173.3445 90.3121) (width 0.2) (layer "F.Cu") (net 12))
 (segment (start 173.3445 56.9428) (end 172.9017 56.5) (width 0.2) (layer "F.Cu") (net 12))
 (segment (start 173.24 97.39) (end 172.0611 96.2111) (width 0.2) (layer "F.Cu") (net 12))
 (segment (start 171 56.5) (end 158.5 56.5) (width 0.2) (layer "B.Cu") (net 12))
 (segment (start 191.75 119.58) (end 191.75 118.6783) (width 0.2) (layer "B.Cu") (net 11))
 (segment (start 174.2083 118.6783) (end 191.75 118.6783) (width 0.2) (layer "B.Cu") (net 11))
 (segment (start 173.24 117.71) (end 174.2083 118.6783) (width 0.2) (layer "B.Cu") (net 11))
 (segment (start 171.85 88.83) (end 171.85 108.7) (width 0.2) (layer "B.Cu") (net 14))
 (segment (start 171.85 108.7) (end 173.24 110.09) (width 0.2) (layer "B.Cu") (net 14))
 (segment (start 174.418 120.25) (end 179.2663 115.4017) (width 0.2) (layer "F.Cu") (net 9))
 (segment (start 179.2663 115.4017) (end 191.75 115.4017) (width 0.2) (layer "F.Cu") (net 9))
 (segment (start 173.24 120.25) (end 174.418 120.25) (width 0.2) (layer "F.Cu") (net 9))
 (segment (start 191.75 114.5) (end 191.75 115.4017) (width 0.2) (layer "F.Cu") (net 9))
 (segment (start 173.24 94.85) (end 177.3483 90.7417) (width 0.2) (layer "F.Cu") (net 19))
 (segment (start 179.25 66.75) (end 177.3483 66.75) (width 0.2) (layer "F.Cu") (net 19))
 (segment (start 177.3483 90.7417) (end 177.3483 66.75) (width 0.2) (layer "F.Cu") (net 19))
 (segment (start 179.25 66.75) (end 191.75 66.75) (width 0.2) (layer "B.Cu") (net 19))
 (segment (start 179.25 51.5) (end 181.1517 51.5) (width 0.2) (layer "F.Cu") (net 17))
 (segment (start 181.1517 78.8472) (end 181.1517 51.5) (width 0.2) (layer "F.Cu") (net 17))
 (segment (start 177.7502 97.9598) (end 177.7502 82.2487) (width 0.2) (layer "F.Cu") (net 17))
 (segment (start 173.24 102.47) (end 177.7502 97.9598) (width 0.2) (layer "F.Cu") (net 17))
 (segment (start 177.7502 82.2487) (end 181.1517 78.8472) (width 0.2) (layer "F.Cu") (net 17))
 (segment (start 179.25 51.5) (end 191.75 51.5) (width 0.2) (layer "B.Cu") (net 17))
 (segment (start 182.9161 73.5144) (end 188.0839 73.5144) (width 0.2) (layer "B.Cu") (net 10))
 (segment (start 188.0839 115.17) (end 188.0839 73.5144) (width 0.2) (layer "B.Cu") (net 10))
 (segment (start 179.25 36.25) (end 172.9017 36.25) (width 0.2) (layer "B.Cu") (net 10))
 (segment (start 177.3498 56.5) (end 177.3483 56.5) (width 0.2) (layer "B.Cu") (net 10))
 (segment (start 189.9539 117.04) (end 188.0839 115.17) (width 0.2) (layer "B.Cu") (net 10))
 (segment (start 158.5 71.5) (end 171 71.5) (width 0.2) (layer "B.Cu") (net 10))
 (segment (start 172.9017 36.25) (end 171 36.25) (width 0.2) (layer "B.Cu") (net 10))
 (segment (start 191.75 56.5) (end 179.25 56.5) (width 0.2) (layer "B.Cu") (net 10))
 (segment (start 191.75 71.75) (end 189.8483 71.75) (width 0.2) (layer "B.Cu") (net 10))
 (segment (start 177.3483 55.9466) (end 172.9017 51.5) (width 0.2) (layer "B.Cu") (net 10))
 (segment (start 177.3483 56.5) (end 177.3483 55.9466) (width 0.2) (layer "B.Cu") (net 10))
 (segment (start 179.25 56.5) (end 177.4492 56.5) (width 0.2) (layer "B.Cu") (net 10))
 (segment (start 188.0839 115.17) (end 173.24 115.17) (width 0.2) (layer "B.Cu") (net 10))
 (segment (start 179.25 71.75) (end 181.1517 71.75) (width 0.2) (layer "B.Cu") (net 10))
 (segment (start 158.5 51.5) (end 171 51.5) (width 0.2) (layer "B.Cu") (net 10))
 (segment (start 191.75 36.25) (end 179.25 36.25) (width 0.2) (layer "B.Cu") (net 10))
 (segment (start 176.3089 71.75) (end 179.25 71.75) (width 0.2) (layer "B.Cu") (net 10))
 (segment (start 171 71.5) (end 172.9017 71.5) (width 0.2) (layer "B.Cu") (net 10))
 (segment (start 188.0839 73.5144) (end 189.8483 71.75) (width 0.2) (layer "B.Cu") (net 10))
 (segment (start 176.0589 57.7909) (end 176.0589 71.5) (width 0.2) (layer "B.Cu") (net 10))
 (segment (start 191.75 117.04) (end 189.9539 117.04) (width 0.2) (layer "B.Cu") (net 10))
 (segment (start 176.0589 71.5) (end 172.9017 71.5) (width 0.2) (layer "B.Cu") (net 10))
 (segment (start 171 36.25) (end 158.5 36.25) (width 0.2) (layer "B.Cu") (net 10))
 (segment (start 181.1517 71.75) (end 182.9161 73.5144) (width 0.2) (layer "B.Cu") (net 10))
 (segment (start 177.4492 56.5) (end 177.3498 56.5) (width 0.2) (layer "B.Cu") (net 10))
 (segment (start 177.3498 56.5) (end 176.0589 57.7909) (width 0.2) (layer "B.Cu") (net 10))
 (segment (start 176.0589 71.5) (end 176.3089 71.75) (width 0.2) (layer "B.Cu") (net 10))
 (segment (start 172.9017 36.25) (end 172.9017 51.5) (width 0.2) (layer "B.Cu") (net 10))
 (segment (start 171 51.5) (end 172.9017 51.5) (width 0.2) (layer "B.Cu") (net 10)))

